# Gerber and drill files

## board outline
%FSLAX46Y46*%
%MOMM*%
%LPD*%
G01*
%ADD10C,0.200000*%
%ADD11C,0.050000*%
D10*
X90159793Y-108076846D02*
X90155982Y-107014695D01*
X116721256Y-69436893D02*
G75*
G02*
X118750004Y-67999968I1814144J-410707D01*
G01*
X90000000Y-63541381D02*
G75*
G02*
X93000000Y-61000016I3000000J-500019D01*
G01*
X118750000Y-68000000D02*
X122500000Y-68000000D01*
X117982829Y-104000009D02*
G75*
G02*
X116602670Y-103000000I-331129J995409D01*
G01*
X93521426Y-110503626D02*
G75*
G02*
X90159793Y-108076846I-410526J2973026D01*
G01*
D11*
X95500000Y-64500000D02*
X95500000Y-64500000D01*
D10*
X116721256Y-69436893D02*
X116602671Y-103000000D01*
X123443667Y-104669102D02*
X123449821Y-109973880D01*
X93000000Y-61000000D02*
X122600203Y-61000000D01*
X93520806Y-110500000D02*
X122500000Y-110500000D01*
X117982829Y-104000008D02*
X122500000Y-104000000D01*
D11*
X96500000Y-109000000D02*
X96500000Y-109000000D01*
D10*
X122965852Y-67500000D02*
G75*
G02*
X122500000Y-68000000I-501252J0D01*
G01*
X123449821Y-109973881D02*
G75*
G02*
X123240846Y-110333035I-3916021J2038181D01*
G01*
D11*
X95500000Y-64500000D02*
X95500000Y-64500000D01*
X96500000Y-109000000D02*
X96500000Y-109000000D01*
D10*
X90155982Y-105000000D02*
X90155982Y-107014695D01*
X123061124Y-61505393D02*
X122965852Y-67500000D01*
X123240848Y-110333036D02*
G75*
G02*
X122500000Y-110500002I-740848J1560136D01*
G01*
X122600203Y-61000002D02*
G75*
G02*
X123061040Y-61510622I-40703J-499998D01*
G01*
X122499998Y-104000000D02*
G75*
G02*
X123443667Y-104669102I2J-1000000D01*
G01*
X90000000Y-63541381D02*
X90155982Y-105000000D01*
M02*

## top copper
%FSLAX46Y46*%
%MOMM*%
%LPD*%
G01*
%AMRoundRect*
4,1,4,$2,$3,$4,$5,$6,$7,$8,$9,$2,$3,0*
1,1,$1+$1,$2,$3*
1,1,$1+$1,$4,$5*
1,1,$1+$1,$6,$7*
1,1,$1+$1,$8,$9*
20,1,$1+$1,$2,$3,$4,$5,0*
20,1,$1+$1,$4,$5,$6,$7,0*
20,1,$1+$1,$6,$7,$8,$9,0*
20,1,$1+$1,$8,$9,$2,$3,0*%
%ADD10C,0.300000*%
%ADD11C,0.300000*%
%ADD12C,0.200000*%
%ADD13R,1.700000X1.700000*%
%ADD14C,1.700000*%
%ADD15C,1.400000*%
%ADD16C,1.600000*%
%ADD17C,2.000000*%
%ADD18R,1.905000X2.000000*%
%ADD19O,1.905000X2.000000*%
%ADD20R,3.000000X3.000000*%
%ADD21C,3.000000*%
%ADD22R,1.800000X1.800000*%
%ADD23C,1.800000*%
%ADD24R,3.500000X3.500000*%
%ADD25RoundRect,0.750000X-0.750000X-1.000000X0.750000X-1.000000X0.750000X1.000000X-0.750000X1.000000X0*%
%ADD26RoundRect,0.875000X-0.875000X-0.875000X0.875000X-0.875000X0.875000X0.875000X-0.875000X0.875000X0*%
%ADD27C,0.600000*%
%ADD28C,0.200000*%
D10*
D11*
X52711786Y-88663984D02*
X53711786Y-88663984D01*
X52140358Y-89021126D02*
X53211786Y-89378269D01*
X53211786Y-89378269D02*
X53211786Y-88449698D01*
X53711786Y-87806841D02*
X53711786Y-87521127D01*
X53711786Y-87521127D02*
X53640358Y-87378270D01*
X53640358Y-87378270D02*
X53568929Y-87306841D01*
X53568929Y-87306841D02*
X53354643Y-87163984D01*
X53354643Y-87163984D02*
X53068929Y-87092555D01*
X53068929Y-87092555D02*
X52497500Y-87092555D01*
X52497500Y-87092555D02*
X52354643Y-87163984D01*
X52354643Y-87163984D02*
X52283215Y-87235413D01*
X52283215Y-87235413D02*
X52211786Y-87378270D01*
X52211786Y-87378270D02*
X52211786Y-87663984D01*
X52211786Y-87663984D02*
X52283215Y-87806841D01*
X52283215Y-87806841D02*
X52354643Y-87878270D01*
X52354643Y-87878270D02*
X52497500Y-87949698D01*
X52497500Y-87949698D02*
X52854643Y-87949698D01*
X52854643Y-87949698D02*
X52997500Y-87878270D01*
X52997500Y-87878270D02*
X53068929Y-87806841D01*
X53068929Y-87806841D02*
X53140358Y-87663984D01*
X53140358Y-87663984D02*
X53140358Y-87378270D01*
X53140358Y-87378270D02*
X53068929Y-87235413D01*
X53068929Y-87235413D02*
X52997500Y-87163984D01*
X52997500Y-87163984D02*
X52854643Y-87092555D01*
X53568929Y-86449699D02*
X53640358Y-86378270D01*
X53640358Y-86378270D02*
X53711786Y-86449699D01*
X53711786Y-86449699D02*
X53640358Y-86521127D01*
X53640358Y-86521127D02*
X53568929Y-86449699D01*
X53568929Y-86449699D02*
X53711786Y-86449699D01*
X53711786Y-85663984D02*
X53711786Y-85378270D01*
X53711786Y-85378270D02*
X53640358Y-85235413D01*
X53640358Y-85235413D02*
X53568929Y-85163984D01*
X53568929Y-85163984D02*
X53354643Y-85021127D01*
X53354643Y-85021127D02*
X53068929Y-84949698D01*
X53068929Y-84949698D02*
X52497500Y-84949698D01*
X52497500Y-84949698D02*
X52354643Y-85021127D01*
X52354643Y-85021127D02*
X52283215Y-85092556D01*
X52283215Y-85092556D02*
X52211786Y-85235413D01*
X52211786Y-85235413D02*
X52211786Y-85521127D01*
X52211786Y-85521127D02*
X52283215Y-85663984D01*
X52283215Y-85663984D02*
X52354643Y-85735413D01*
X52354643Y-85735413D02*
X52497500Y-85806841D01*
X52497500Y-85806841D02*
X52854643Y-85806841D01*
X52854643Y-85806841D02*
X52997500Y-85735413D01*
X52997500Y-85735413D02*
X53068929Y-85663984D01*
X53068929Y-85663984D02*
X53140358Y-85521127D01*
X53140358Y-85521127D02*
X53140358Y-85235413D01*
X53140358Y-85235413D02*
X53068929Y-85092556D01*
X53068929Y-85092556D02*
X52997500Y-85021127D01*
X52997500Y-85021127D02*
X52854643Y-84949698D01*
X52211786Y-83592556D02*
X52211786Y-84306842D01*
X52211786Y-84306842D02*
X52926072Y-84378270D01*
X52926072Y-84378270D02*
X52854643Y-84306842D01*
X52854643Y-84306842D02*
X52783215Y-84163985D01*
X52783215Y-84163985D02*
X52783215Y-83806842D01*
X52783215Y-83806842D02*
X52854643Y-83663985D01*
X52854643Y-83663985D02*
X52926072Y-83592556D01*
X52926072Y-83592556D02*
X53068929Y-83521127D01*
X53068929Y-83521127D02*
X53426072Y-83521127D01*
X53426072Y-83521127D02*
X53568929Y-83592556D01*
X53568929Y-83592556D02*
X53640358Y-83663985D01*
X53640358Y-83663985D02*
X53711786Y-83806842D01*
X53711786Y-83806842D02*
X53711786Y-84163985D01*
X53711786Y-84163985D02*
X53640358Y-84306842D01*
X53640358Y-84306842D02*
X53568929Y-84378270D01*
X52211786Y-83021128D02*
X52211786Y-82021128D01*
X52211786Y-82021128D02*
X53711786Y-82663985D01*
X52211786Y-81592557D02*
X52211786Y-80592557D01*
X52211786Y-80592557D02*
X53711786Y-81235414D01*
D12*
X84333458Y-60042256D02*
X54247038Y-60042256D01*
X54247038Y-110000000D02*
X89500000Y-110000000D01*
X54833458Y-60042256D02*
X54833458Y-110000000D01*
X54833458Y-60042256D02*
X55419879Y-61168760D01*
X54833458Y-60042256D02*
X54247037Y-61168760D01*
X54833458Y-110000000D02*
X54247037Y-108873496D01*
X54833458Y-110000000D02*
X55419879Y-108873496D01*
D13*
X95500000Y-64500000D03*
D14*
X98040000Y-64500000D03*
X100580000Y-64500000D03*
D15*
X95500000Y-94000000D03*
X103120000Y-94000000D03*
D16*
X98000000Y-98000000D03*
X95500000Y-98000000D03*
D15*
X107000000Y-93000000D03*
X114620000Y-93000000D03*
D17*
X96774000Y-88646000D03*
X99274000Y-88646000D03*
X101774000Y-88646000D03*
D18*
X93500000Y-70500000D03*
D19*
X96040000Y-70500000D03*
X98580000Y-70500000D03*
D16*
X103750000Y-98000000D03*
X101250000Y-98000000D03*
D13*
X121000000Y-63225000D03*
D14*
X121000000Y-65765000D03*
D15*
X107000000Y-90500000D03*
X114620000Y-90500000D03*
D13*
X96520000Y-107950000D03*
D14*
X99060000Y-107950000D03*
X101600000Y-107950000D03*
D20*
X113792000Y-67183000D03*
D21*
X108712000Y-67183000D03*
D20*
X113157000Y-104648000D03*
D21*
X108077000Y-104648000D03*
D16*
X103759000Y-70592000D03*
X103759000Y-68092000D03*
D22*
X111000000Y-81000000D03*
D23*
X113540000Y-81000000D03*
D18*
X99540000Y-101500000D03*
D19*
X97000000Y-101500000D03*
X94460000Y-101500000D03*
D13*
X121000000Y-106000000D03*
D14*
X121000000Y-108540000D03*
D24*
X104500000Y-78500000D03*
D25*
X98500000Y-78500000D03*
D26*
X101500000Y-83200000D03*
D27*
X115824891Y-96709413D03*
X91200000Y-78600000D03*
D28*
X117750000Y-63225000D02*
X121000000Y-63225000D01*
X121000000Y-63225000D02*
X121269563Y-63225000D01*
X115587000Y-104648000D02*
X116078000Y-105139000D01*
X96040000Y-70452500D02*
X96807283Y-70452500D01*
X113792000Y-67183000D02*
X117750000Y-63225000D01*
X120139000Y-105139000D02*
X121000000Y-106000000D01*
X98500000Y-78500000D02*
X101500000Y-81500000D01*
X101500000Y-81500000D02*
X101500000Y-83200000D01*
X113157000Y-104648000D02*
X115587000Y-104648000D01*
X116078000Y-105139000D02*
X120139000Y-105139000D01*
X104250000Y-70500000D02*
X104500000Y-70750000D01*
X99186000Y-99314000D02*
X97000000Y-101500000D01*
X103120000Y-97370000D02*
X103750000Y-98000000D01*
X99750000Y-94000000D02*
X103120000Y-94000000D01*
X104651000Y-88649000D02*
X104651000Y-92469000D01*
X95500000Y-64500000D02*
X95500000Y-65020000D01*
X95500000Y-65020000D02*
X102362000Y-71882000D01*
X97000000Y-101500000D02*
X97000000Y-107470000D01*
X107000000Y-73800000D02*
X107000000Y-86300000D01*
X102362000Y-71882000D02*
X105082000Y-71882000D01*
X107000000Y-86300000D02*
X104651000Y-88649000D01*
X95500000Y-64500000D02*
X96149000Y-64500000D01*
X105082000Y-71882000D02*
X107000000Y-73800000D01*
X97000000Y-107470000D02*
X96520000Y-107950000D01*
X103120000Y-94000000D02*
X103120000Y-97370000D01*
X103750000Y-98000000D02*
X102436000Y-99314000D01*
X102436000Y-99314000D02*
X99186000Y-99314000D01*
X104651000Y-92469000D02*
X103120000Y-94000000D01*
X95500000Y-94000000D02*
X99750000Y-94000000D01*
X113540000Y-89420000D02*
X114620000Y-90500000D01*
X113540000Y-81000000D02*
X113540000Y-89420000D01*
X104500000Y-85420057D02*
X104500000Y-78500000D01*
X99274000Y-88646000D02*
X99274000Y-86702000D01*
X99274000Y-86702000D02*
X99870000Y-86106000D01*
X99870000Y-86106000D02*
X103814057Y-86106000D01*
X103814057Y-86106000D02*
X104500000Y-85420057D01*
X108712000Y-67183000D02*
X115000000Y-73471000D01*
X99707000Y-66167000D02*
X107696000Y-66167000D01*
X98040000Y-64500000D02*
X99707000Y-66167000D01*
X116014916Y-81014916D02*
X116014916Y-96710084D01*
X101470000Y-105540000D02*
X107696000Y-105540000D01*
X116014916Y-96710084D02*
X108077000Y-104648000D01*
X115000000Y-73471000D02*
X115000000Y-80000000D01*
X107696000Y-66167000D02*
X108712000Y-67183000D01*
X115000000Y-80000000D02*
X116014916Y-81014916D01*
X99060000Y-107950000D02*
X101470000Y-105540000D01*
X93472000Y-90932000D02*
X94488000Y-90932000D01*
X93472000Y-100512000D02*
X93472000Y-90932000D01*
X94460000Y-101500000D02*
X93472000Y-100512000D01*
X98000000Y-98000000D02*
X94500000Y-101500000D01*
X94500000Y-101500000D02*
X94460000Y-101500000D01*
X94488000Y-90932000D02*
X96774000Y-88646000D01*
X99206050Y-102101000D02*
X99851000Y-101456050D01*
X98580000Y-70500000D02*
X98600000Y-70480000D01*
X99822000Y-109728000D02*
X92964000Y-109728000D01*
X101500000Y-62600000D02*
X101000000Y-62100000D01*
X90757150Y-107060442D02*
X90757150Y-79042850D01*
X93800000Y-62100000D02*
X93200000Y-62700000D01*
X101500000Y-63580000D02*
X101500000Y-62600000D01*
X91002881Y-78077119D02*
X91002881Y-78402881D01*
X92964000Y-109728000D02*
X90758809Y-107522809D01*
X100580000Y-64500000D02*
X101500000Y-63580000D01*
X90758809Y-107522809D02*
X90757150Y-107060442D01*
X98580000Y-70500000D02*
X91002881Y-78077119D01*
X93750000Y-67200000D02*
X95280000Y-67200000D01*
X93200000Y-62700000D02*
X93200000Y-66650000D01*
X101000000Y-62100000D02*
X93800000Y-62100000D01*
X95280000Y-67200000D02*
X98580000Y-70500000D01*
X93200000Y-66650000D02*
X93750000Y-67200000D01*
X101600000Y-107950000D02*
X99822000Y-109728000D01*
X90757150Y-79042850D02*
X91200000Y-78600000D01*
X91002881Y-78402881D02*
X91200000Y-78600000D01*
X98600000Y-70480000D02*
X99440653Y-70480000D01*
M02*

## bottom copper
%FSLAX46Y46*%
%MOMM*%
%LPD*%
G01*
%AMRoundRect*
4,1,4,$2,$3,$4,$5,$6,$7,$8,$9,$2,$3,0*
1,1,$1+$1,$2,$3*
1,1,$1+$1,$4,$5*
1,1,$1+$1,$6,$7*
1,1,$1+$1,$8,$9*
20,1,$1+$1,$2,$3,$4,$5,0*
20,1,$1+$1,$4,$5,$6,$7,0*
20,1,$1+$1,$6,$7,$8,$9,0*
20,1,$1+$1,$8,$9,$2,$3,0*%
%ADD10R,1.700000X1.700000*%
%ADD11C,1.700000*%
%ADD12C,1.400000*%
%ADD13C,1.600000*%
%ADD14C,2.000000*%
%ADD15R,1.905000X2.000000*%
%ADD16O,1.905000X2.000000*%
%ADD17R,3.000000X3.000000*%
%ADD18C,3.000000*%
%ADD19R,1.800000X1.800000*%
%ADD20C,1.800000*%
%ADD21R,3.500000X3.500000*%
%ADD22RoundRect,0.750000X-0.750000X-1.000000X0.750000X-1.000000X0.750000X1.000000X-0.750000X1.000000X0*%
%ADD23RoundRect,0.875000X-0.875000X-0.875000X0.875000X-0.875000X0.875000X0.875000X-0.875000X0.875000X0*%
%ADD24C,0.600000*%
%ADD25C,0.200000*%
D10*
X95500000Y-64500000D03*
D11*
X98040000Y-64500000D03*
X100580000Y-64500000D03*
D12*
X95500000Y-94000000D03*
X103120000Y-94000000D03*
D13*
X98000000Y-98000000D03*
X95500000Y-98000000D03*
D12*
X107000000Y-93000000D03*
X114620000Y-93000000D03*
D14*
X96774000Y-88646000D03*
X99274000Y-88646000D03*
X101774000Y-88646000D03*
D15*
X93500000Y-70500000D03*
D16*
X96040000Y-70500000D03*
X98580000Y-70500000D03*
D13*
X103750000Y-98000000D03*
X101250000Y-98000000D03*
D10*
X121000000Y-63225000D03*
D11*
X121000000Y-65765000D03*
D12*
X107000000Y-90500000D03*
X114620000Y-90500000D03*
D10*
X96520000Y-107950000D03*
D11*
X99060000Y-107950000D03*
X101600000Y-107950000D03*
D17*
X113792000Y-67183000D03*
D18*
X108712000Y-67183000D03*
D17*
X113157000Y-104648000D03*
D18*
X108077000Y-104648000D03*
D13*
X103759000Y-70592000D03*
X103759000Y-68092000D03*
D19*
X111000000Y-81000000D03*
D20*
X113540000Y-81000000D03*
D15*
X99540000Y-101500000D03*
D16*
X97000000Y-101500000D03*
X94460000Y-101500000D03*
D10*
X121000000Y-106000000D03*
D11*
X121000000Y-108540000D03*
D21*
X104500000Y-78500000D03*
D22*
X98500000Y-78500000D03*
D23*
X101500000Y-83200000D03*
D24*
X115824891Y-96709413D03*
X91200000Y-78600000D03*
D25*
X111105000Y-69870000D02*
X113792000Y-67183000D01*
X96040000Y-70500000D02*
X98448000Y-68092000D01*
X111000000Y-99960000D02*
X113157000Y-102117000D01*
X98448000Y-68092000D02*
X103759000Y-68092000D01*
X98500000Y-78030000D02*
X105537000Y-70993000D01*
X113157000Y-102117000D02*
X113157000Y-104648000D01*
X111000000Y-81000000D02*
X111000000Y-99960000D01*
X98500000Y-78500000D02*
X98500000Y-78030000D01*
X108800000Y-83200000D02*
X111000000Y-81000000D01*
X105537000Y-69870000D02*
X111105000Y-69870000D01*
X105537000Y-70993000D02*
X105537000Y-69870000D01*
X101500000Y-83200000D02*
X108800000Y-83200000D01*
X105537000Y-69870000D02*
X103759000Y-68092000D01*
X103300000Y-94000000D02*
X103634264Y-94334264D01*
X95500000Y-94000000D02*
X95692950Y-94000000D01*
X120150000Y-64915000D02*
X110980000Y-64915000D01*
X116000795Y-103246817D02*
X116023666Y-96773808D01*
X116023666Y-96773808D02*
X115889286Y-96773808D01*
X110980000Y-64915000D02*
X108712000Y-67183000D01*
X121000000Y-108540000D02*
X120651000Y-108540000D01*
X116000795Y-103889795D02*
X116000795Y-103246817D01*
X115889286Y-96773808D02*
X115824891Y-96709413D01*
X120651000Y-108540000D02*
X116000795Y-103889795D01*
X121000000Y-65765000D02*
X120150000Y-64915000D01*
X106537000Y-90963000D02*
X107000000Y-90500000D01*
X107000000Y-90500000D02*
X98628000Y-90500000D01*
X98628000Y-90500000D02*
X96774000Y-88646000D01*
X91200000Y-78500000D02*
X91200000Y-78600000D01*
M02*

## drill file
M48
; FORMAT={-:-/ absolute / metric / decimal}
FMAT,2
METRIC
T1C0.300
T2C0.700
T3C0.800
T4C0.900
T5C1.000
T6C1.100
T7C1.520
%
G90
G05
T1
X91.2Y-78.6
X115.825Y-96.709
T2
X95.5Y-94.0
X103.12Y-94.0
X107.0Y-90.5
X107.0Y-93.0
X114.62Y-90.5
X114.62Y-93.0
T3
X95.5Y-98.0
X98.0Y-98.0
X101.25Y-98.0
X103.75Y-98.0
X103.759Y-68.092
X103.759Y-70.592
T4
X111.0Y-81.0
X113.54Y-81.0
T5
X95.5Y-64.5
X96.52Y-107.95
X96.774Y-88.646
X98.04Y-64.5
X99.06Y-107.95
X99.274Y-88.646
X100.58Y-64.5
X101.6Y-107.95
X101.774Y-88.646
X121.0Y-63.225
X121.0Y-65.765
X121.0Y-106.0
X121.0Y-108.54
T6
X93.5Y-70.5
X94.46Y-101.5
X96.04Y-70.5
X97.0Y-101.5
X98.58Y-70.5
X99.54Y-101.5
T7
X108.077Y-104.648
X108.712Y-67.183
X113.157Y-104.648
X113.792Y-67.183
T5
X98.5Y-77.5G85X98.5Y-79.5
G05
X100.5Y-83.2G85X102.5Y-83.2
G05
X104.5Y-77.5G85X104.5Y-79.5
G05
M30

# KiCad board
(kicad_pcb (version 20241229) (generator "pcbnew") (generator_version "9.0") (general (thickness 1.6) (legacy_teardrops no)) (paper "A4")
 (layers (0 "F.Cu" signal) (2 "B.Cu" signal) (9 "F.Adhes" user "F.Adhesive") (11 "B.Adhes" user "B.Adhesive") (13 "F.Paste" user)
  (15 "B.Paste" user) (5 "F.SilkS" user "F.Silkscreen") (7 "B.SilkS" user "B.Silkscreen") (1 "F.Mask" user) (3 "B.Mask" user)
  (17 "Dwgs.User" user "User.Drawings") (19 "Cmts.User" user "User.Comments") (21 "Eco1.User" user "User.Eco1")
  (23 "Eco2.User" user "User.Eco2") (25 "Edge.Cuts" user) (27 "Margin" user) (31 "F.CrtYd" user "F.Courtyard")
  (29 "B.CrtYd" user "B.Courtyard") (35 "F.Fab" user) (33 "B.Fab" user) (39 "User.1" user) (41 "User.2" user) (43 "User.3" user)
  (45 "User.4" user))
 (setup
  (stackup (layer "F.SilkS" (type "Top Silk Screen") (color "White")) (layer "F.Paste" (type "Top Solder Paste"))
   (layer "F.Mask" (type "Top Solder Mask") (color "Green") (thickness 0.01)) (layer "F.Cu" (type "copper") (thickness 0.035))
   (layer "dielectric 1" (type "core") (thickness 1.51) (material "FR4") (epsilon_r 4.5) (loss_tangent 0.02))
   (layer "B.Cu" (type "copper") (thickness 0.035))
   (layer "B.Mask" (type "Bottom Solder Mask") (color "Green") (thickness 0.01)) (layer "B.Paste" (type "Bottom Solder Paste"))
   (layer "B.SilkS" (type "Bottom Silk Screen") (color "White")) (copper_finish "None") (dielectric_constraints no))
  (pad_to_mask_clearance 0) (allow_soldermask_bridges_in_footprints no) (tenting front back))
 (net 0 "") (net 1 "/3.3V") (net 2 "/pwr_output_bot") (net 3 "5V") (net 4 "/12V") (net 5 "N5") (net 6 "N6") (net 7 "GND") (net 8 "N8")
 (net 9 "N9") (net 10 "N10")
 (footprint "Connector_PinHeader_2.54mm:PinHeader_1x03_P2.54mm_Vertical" (layer "F.Cu") (at 95.5 64.5 90)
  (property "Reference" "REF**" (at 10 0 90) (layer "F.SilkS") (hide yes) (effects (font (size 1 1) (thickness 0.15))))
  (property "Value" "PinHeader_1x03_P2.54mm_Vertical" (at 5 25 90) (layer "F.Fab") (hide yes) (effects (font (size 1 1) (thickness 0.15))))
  (pad "1" thru_hole rect (at 0 0 90) (size 1.7 1.7) (drill 1) (layers "*.Cu" "*.Mask") (remove_unused_layers no) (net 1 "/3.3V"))
  (pad "2" thru_hole circle (at 0 2.54 90) (size 1.7 1.7) (drill 1) (layers "*.Cu" "*.Mask") (remove_unused_layers no)
   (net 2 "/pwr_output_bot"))
  (pad "3" thru_hole circle (at 0 5.08 90) (size 1.7 1.7) (drill 1) (layers "*.Cu" "*.Mask") (remove_unused_layers no) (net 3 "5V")))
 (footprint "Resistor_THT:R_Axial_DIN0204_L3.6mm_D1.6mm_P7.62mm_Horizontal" (layer "F.Cu") (at 95.5 94)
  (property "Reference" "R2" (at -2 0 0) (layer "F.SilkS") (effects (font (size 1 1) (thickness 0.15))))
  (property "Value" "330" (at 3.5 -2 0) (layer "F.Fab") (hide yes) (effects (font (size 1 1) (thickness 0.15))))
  (pad "1" thru_hole circle (at 0 0) (size 1.4 1.4) (drill 0.7) (layers "*.Cu" "*.Mask") (remove_unused_layers no) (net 1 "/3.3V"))
  (pad "2" thru_hole circle (at 7.62 0) (size 1.4 1.4) (drill 0.7) (layers "*.Cu" "*.Mask") (remove_unused_layers no) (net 1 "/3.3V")))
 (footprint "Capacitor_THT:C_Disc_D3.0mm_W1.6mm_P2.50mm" (layer "F.Cu") (at 95.5 98)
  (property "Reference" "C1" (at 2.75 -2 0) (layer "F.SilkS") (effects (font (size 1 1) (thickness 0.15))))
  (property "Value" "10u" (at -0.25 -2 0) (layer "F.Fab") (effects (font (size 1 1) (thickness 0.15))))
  (pad "1" thru_hole circle (at 2.5 0) (size 1.6 1.6) (drill 0.8) (layers "*.Cu" "*.Mask") (remove_unused_layers no) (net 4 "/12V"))
  (pad "2" thru_hole circle (at 0 0) (size 1.6 1.6) (drill 0.8) (layers "*.Cu" "*.Mask") (remove_unused_layers no)))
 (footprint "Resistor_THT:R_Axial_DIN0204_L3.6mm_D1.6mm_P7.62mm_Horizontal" (layer "F.Cu") (at 107 93)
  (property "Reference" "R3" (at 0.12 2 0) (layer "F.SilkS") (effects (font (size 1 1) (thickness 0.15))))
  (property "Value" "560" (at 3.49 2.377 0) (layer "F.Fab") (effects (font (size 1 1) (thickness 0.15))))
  (pad "1" thru_hole circle (at 0 0) (size 1.4 1.4) (drill 0.7) (layers "*.Cu" "*.Mask") (remove_unused_layers no))
  (pad "2" thru_hole circle (at 7.62 0) (size 1.4 1.4) (drill 0.7) (layers "*.Cu" "*.Mask") (remove_unused_layers no)))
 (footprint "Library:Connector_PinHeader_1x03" (layer "F.Cu") (at 98.774 92.146)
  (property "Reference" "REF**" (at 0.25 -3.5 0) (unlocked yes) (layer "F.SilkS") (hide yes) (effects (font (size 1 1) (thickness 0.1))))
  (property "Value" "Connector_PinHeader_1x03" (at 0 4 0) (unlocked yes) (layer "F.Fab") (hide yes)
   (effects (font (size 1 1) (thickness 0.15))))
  (pad "1" thru_hole circle (at -2 -3.5) (size 2 2) (drill 1) (layers "*.Cu" "*.Mask") (remove_unused_layers no) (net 4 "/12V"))
  (pad "2" thru_hole circle (at 0.5 -3.5) (size 2 2) (drill 1) (layers "*.Cu" "*.Mask") (remove_unused_layers no) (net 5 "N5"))
  (pad "3" thru_hole circle (at 3 -3.5) (size 2 2) (drill 1) (layers "*.Cu" "*.Mask") (remove_unused_layers no)))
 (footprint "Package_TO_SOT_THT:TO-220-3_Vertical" (layer "F.Cu") (at 93.5 70.5)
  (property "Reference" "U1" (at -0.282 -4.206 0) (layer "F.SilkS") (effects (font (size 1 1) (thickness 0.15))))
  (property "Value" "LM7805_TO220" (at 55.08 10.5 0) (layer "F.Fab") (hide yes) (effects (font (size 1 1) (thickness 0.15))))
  (pad "1" thru_hole rect (at 0 0) (size 1.905 2) (drill 1.1) (layers "*.Cu" "*.Mask") (remove_unused_layers no) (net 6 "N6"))
  (pad "2" thru_hole oval (at 2.54 0) (size 1.905 2) (drill 1.1) (layers "*.Cu" "*.Mask") (remove_unused_layers no) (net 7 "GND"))
  (pad "3" thru_hole oval (at 5.08 0) (size 1.905 2) (drill 1.1) (layers "*.Cu" "*.Mask") (remove_unused_layers no) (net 3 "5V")))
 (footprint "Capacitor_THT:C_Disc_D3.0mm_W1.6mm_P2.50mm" (layer "F.Cu") (at 101.25 98)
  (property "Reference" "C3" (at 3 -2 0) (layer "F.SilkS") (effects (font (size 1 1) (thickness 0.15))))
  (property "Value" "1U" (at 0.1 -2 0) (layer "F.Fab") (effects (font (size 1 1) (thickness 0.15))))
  (pad "1" thru_hole circle (at 2.5 0) (size 1.6 1.6) (drill 0.8) (layers "*.Cu" "*.Mask") (remove_unused_layers no) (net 1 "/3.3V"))
  (pad "2" thru_hole circle (at 0 0) (size 1.6 1.6) (drill 0.8) (layers "*.Cu" "*.Mask") (remove_unused_layers no)))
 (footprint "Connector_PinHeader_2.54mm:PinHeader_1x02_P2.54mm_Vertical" (layer "F.Cu") (at 121 63.225)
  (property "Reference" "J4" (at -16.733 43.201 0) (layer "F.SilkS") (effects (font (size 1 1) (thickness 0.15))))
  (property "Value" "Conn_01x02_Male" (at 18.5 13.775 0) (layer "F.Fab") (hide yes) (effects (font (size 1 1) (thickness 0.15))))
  (pad "1" thru_hole rect (at 0 0) (size 1.7 1.7) (drill 1) (layers "*.Cu" "*.Mask") (remove_unused_layers no) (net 7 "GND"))
  (pad "2" thru_hole circle (at 0 2.54) (size 1.7 1.7) (drill 1) (layers "*.Cu" "*.Mask") (remove_unused_layers no)
   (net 2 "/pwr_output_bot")))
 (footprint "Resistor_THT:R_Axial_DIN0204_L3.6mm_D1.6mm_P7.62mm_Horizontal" (layer "F.Cu") (at 107 90.5)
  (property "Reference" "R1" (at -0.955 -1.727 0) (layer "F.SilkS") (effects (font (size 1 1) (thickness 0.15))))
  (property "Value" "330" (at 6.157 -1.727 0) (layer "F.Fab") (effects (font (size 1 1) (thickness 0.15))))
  (pad "1" thru_hole circle (at 0 0) (size 1.4 1.4) (drill 0.7) (layers "*.Cu" "*.Mask") (remove_unused_layers no) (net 4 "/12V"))
  (pad "2" thru_hole circle (at 7.62 0) (size 1.4 1.4) (drill 0.7) (layers "*.Cu" "*.Mask") (remove_unused_layers no) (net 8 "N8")))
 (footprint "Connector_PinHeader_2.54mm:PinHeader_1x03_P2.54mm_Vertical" (layer "F.Cu") (at 96.52 107.95 90)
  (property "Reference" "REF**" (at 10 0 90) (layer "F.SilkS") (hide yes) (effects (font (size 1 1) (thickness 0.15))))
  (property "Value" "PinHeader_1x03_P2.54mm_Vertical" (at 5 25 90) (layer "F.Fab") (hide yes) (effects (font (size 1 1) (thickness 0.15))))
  (pad "1" thru_hole rect (at 0 0 90) (size 1.7 1.7) (drill 1) (layers "*.Cu" "*.Mask") (remove_unused_layers no) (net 1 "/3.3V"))
  (pad "2" thru_hole circle (at 0 2.54 90) (size 1.7 1.7) (drill 1) (layers "*.Cu" "*.Mask") (remove_unused_layers no)
   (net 2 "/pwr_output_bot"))
  (pad "3" thru_hole circle (at 0 5.08 90) (size 1.7 1.7) (drill 1) (layers "*.Cu" "*.Mask") (remove_unused_layers no) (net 3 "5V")))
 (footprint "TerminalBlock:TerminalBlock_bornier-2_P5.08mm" (layer "F.Cu") (at 113.792 67.183 180)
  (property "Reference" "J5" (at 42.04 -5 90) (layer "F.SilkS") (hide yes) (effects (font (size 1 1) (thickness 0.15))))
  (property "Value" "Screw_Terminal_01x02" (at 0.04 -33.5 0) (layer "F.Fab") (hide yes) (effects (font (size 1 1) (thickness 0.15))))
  (pad "1" thru_hole rect (at 0 0 180) (size 3 3) (drill 1.52) (layers "*.Cu" "*.Mask") (remove_unused_layers no) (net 7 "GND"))
  (pad "2" thru_hole circle (at 5.08 0 180) (size 3 3) (drill 1.52) (layers "*.Cu" "*.Mask") (remove_unused_layers no)
   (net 2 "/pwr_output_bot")))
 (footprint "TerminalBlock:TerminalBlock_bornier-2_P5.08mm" (layer "F.Cu") (at 113.157 104.648 180)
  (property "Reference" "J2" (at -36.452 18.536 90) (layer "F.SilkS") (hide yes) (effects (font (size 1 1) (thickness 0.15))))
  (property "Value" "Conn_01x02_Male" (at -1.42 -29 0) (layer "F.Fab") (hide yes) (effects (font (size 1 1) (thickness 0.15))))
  (pad "1" thru_hole rect (at 0 0 180) (size 3 3) (drill 1.52) (layers "*.Cu" "*.Mask") (remove_unused_layers no) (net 7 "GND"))
  (pad "2" thru_hole circle (at 5.08 0 180) (size 3 3) (drill 1.52) (layers "*.Cu" "*.Mask") (remove_unused_layers no)
   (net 2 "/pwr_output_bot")))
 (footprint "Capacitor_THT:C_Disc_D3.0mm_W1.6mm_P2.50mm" (layer "F.Cu") (at 103.759 70.592 90)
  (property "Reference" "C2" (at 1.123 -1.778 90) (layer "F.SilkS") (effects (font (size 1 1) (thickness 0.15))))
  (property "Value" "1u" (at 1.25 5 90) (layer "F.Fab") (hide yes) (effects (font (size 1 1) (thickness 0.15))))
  (pad "1" thru_hole circle (at 0 0 90) (size 1.6 1.6) (drill 0.8) (layers "*.Cu" "*.Mask") (remove_unused_layers no) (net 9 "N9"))
  (pad "2" thru_hole circle (at 2.5 0 90) (size 1.6 1.6) (drill 0.8) (layers "*.Cu" "*.Mask") (remove_unused_layers no) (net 7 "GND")))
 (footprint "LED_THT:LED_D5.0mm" (layer "F.Cu") (at 111 81)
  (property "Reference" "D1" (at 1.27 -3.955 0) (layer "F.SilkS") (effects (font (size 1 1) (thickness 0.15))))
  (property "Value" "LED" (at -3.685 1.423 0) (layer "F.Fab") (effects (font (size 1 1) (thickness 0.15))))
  (pad "1" thru_hole rect (at 0 0) (size 1.8 1.8) (drill 0.9) (layers "*.Cu" "*.Mask") (remove_unused_layers no) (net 7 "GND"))
  (pad "2" thru_hole circle (at 2.54 0) (size 1.8 1.8) (drill 0.9) (layers "*.Cu" "*.Mask") (remove_unused_layers no) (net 8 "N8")))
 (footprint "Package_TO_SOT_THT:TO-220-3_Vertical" (layer "F.Cu") (at 99.54 101.5 180)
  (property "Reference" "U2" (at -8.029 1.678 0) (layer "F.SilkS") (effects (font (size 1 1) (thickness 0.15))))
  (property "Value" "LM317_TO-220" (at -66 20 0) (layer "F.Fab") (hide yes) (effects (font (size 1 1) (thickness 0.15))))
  (pad "1" thru_hole rect (at 0 0 180) (size 1.905 2) (drill 1.1) (layers "*.Cu" "*.Mask") (remove_unused_layers no) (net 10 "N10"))
  (pad "2" thru_hole oval (at 2.54 0 180) (size 1.905 2) (drill 1.1) (layers "*.Cu" "*.Mask") (remove_unused_layers no) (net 1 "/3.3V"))
  (pad "3" thru_hole oval (at 5.08 0 180) (size 1.905 2) (drill 1.1) (layers "*.Cu" "*.Mask") (remove_unused_layers no) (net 4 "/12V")))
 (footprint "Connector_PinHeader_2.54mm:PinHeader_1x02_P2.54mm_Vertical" (layer "F.Cu") (at 121 106)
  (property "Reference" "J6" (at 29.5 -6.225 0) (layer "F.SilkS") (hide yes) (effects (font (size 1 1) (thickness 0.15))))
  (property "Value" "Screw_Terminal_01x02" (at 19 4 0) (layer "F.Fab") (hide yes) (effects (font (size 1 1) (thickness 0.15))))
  (pad "1" thru_hole rect (at 0 0) (size 1.7 1.7) (drill 1) (layers "*.Cu" "*.Mask") (remove_unused_layers no) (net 7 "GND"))
  (pad "2" thru_hole circle (at 0 2.54) (size 1.7 1.7) (drill 1) (layers "*.Cu" "*.Mask") (remove_unused_layers no)
   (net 2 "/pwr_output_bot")))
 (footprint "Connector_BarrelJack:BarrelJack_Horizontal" (layer "F.Cu") (at 104.5 78.5)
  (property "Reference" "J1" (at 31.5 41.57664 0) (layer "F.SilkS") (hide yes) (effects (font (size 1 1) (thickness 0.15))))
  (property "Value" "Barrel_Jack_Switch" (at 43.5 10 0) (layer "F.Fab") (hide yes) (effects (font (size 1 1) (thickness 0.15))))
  (pad "1" thru_hole rect (at 0 0) (size 3.5 3.5) (drill oval 1 3) (layers "*.Cu" "*.Mask") (remove_unused_layers no) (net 5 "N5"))
  (pad "2" thru_hole roundrect (at -6 0) (size 3 3.5) (drill oval 1 3) (layers "*.Cu" "*.Mask") (remove_unused_layers no)
   (roundrect_rratio 0.25) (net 7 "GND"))
  (pad "3" thru_hole roundrect (at -3 4.7) (size 3.5 3.5) (drill oval 3 1) (layers "*.Cu" "*.Mask") (remove_unused_layers no)
   (roundrect_rratio 0.25) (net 7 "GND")))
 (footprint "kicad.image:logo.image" (layer "B.Cu") (at 110.49 86.106 180)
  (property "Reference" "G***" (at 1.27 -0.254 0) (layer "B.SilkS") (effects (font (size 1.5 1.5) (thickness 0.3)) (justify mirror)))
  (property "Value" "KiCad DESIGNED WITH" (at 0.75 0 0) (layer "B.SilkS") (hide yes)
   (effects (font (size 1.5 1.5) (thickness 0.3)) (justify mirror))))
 (gr_line (start 90.159793 108.076846) (end 90.155982 107.014695) (stroke (width 0.2) (type solid)) (layer "Edge.Cuts"))
 (gr_arc (start 116.721256 69.436893) (mid 117.460312 68.329729) (end 118.75 68) (stroke (width 0.2) (type solid)) (layer "Edge.Cuts"))
 (gr_arc (start 90 63.541381) (mid 91.034128 61.720746) (end 93 61) (stroke (width 0.2) (type solid)) (layer "Edge.Cuts"))
 (gr_line (start 118.75 68) (end 122.5 68) (stroke (width 0.2) (type solid)) (layer "Edge.Cuts"))
 (gr_arc (start 117.982829 104.000009) (mid 117.036207 103.854071) (end 116.60267 103) (stroke (width 0.2) (type solid)) (layer "Edge.Cuts"))
 (gr_arc (start 93.521426 110.503626) (mid 91.354212 109.964005) (end 90.159793 108.076846) (stroke (width 0.2) (type solid))
  (layer "Edge.Cuts"))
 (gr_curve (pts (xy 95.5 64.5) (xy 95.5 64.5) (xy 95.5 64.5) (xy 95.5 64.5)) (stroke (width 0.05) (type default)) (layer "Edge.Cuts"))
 (gr_line (start 116.721256 69.436893) (end 116.602671 103) (stroke (width 0.2) (type solid)) (layer "Edge.Cuts"))
 (gr_line (start 123.443667 104.669102) (end 123.449821 109.97388) (stroke (width 0.2) (type solid)) (layer "Edge.Cuts"))
 (gr_line (start 93 61) (end 122.600203 61) (stroke (width 0.2) (type solid)) (layer "Edge.Cuts"))
 (gr_line (start 93.520806 110.5) (end 122.5 110.5) (stroke (width 0.2) (type solid)) (layer "Edge.Cuts"))
 (gr_line (start 117.982829 104.000008) (end 122.5 104) (stroke (width 0.2) (type solid)) (layer "Edge.Cuts"))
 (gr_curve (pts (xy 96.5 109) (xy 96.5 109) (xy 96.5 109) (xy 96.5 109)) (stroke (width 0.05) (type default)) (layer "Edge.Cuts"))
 (gr_arc (start 122.965852 67.5) (mid 122.831341 67.841694) (end 122.5 68) (stroke (width 0.2) (type solid)) (layer "Edge.Cuts"))
 (gr_arc (start 123.449821 109.973881) (mid 123.34956 110.155917) (end 123.240843 110.333033) (stroke (width 0.2) (type solid))
  (layer "Edge.Cuts"))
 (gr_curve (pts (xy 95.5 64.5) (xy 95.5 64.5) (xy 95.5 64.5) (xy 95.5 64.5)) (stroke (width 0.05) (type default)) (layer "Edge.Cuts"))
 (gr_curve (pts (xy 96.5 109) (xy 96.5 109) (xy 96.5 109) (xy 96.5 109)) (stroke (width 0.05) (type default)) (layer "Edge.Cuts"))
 (gr_line (start 90.155982 105) (end 90.155982 107.014695) (stroke (width 0.2) (type solid)) (layer "Edge.Cuts"))
 (gr_line (start 123.061124 61.505393) (end 122.965852 67.5) (stroke (width 0.2) (type solid)) (layer "Edge.Cuts"))
 (gr_arc (start 123.240848 110.333036) (mid 122.879715 110.457742) (end 122.5 110.5) (stroke (width 0.2) (type solid)) (layer "Edge.Cuts"))
 (gr_arc (start 122.600203 61.000002) (mid 122.931911 61.163898) (end 123.06104 61.510622) (stroke (width 0.2) (type solid))
  (layer "Edge.Cuts"))
 (gr_arc (start 122.499998 104) (mid 123.078403 104.184249) (end 123.443667 104.669102) (stroke (width 0.2) (type solid))
  (layer "Edge.Cuts"))
 (gr_line (start 90 63.541381) (end 90.155982 105) (stroke (width 0.2) (type solid)) (layer "Edge.Cuts"))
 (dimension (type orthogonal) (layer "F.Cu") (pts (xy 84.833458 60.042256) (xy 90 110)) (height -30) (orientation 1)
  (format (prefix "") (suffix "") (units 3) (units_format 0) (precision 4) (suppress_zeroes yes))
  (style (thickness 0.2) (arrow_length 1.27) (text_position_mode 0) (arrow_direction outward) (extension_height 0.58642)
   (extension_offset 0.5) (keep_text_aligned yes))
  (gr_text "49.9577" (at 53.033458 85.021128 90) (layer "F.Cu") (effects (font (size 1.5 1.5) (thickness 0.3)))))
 (segment (start 117.75 63.225) (end 121 63.225) (width 0.2) (layer "F.Cu") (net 7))
 (segment (start 121 63.225) (end 121.269563 63.225) (width 0.2) (layer "F.Cu") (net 7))
 (segment (start 115.587 104.648) (end 116.078 105.139) (width 0.2) (layer "F.Cu") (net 7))
 (segment (start 96.04 70.4525) (end 96.807283 70.4525) (width 0.2) (layer "F.Cu") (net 7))
 (segment (start 113.792 67.183) (end 117.75 63.225) (width 0.2) (layer "F.Cu") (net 7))
 (segment (start 120.139 105.139) (end 121 106) (width 0.2) (layer "F.Cu") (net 7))
 (segment (start 98.5 78.5) (end 101.5 81.5) (width 0.2) (layer "F.Cu") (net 7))
 (segment (start 101.5 81.5) (end 101.5 83.2) (width 0.2) (layer "F.Cu") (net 7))
 (segment (start 113.157 104.648) (end 115.587 104.648) (width 0.2) (layer "F.Cu") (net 7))
 (segment (start 116.078 105.139) (end 120.139 105.139) (width 0.2) (layer "F.Cu") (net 7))
 (segment (start 111.105 69.87) (end 113.792 67.183) (width 0.2) (layer "B.Cu") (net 7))
 (segment (start 96.04 70.5) (end 98.448 68.092) (width 0.2) (layer "B.Cu") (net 7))
 (segment (start 111 99.96) (end 113.157 102.117) (width 0.2) (layer "B.Cu") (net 7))
 (segment (start 98.448 68.092) (end 103.759 68.092) (width 0.2) (layer "B.Cu") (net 7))
 (segment (start 98.5 78.03) (end 105.537 70.993) (width 0.2) (layer "B.Cu") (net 7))
 (segment (start 113.157 102.117) (end 113.157 104.648) (width 0.2) (layer "B.Cu") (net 7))
 (segment (start 111 81) (end 111 99.96) (width 0.2) (layer "B.Cu") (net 7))
 (segment (start 98.5 78.5) (end 98.5 78.03) (width 0.2) (layer "B.Cu") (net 7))
 (segment (start 108.8 83.2) (end 111 81) (width 0.2) (layer "B.Cu") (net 7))
 (segment (start 105.537 69.87) (end 111.105 69.87) (width 0.2) (layer "B.Cu") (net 7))
 (segment (start 105.537 70.993) (end 105.537 69.87) (width 0.2) (layer "B.Cu") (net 7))
 (segment (start 101.5 83.2) (end 108.8 83.2) (width 0.2) (layer "B.Cu") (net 7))
 (segment (start 105.537 69.87) (end 103.759 68.092) (width 0.2) (layer "B.Cu") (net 7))
 (segment (start 104.25 70.5) (end 104.5 70.75) (width 0.2) (layer "F.Cu") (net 9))
 (segment (start 99.186 99.314) (end 97 101.5) (width 0.2) (layer "F.Cu") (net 1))
 (segment (start 103.12 97.37) (end 103.75 98) (width 0.2) (layer "F.Cu") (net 1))
 (segment (start 99.75 94) (end 103.12 94) (width 0.2) (layer "F.Cu") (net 1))
 (segment (start 104.651 88.649) (end 104.651 92.469) (width 0.2) (layer "F.Cu") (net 1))
 (segment (start 95.5 64.5) (end 95.5 65.02) (width 0.2) (layer "F.Cu") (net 1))
 (segment (start 95.5 65.02) (end 102.362 71.882) (width 0.2) (layer "F.Cu") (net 1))
 (segment (start 97 101.5) (end 97 107.47) (width 0.2) (layer "F.Cu") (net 1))
 (segment (start 107 73.8) (end 107 86.3) (width 0.2) (layer "F.Cu") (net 1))
 (segment (start 102.362 71.882) (end 105.082 71.882) (width 0.2) (layer "F.Cu") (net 1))
 (segment (start 107 86.3) (end 104.651 88.649) (width 0.2) (layer "F.Cu") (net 1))
 (segment (start 95.5 64.5) (end 96.149 64.5) (width 0.2) (layer "F.Cu") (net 1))
 (segment (start 105.082 71.882) (end 107 73.8) (width 0.2) (layer "F.Cu") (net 1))
 (segment (start 97 107.47) (end 96.52 107.95) (width 0.2) (layer "F.Cu") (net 1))
 (segment (start 103.12 94) (end 103.12 97.37) (width 0.2) (layer "F.Cu") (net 1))
 (segment (start 103.75 98) (end 102.436 99.314) (width 0.2) (layer "F.Cu") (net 1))
 (segment (start 102.436 99.314) (end 99.186 99.314) (width 0.2) (layer "F.Cu") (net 1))
 (segment (start 104.651 92.469) (end 103.12 94) (width 0.2) (layer "F.Cu") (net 1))
 (segment (start 95.5 94) (end 99.75 94) (width 0.2) (layer "F.Cu") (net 1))
 (segment (start 103.3 94) (end 103.634264 94.334264) (width 0.2) (layer "B.Cu") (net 1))
 (segment (start 95.5 94) (end 95.69295 94) (width 0.2) (layer "B.Cu") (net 1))
 (segment (start 113.54 89.42) (end 114.62 90.5) (width 0.2) (layer "F.Cu") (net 8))
 (segment (start 113.54 81) (end 113.54 89.42) (width 0.2) (layer "F.Cu") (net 8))
 (segment (start 104.5 85.420057) (end 104.5 78.5) (width 0.2) (layer "F.Cu") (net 5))
 (segment (start 99.274 88.646) (end 99.274 86.702) (width 0.2) (layer "F.Cu") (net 5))
 (segment (start 99.274 86.702) (end 99.87 86.106) (width 0.2) (layer "F.Cu") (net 5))
 (segment (start 99.87 86.106) (end 103.814057 86.106) (width 0.2) (layer "F.Cu") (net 5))
 (segment (start 103.814057 86.106) (end 104.5 85.420057) (width 0.2) (layer "F.Cu") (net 5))
 (segment (start 108.712 67.183) (end 115 73.471) (width 0.2) (layer "F.Cu") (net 2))
 (segment (start 99.707 66.167) (end 107.696 66.167) (width 0.2) (layer "F.Cu") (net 2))
 (segment (start 98.04 64.5) (end 99.707 66.167) (width 0.2) (layer "F.Cu") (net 2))
 (segment (start 116.014916 81.014916) (end 116.014916 96.710084) (width 0.2) (layer "F.Cu") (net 2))
 (segment (start 101.47 105.54) (end 107.696 105.54) (width 0.2) (layer "F.Cu") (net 2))
 (segment (start 116.014916 96.710084) (end 108.077 104.648) (width 0.2) (layer "F.Cu") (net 2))
 (segment (start 115 73.471) (end 115 80) (width 0.2) (layer "F.Cu") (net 2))
 (segment (start 107.696 66.167) (end 108.712 67.183) (width 0.2) (layer "F.Cu") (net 2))
 (segment (start 115 80) (end 116.014916 81.014916) (width 0.2) (layer "F.Cu") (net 2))
 (segment (start 99.06 107.95) (end 101.47 105.54) (width 0.2) (layer "F.Cu") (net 2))
 (via (at 115.824891 96.709413) (size 0.6) (drill 0.3) (layers "F.Cu" "B.Cu") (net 2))
 (segment (start 120.15 64.915) (end 110.98 64.915) (width 0.2) (layer "B.Cu") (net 2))
 (segment (start 116.000795 103.246817) (end 116.023666 96.773808) (width 0.2) (layer "B.Cu") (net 2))
 (segment (start 116.023666 96.773808) (end 115.889286 96.773808) (width 0.2) (layer "B.Cu") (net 2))
 (segment (start 110.98 64.915) (end 108.712 67.183) (width 0.2) (layer "B.Cu") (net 2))
 (segment (start 121 108.54) (end 120.651 108.54) (width 0.2) (layer "B.Cu") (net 2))
 (segment (start 116.000795 103.889795) (end 116.000795 103.246817) (width 0.2) (layer "B.Cu") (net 2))
 (segment (start 115.889286 96.773808) (end 115.824891 96.709413) (width 0.2) (layer "B.Cu") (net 2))
 (segment (start 120.651 108.54) (end 116.000795 103.889795) (width 0.2) (layer "B.Cu") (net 2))
 (segment (start 121 65.765) (end 120.15 64.915) (width 0.2) (layer "B.Cu") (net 2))
 (segment (start 93.472 90.932) (end 94.488 90.932) (width 0.2) (layer "F.Cu") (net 4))
 (segment (start 93.472 100.512) (end 93.472 90.932) (width 0.2) (layer "F.Cu") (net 4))
 (segment (start 94.46 101.5) (end 93.472 100.512) (width 0.2) (layer "F.Cu") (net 4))
 (segment (start 98 98) (end 94.5 101.5) (width 0.2) (layer "F.Cu") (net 4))
 (segment (start 94.5 101.5) (end 94.46 101.5) (width 0.2) (layer "F.Cu") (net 4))
 (segment (start 94.488 90.932) (end 96.774 88.646) (width 0.2) (layer "F.Cu") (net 4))
 (segment (start 106.537 90.963) (end 107 90.5) (width 0.2) (layer "B.Cu") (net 4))
 (segment (start 107 90.5) (end 98.628 90.5) (width 0.2) (layer "B.Cu") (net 4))
 (segment (start 98.628 90.5) (end 96.774 88.646) (width 0.2) (layer "B.Cu") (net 4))
 (segment (start 99.20605 102.101) (end 99.851 101.45605) (width 0.2) (layer "F.Cu") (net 10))
 (segment (start 98.58 70.5) (end 98.6 70.48) (width 0.2) (layer "F.Cu") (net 3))
 (segment (start 99.822 109.728) (end 92.964 109.728) (width 0.2) (layer "F.Cu") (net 3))
 (segment (start 101.5 62.6) (end 101 62.1) (width 0.2) (layer "F.Cu") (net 3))
 (segment (start 90.75715 107.060442) (end 90.75715 79.04285) (width 0.2) (layer "F.Cu") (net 3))
 (segment (start 93.8 62.1) (end 93.2 62.7) (width 0.2) (layer "F.Cu") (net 3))
 (segment (start 101.5 63.58) (end 101.5 62.6) (width 0.2) (layer "F.Cu") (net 3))
 (segment (start 91.002881 78.077119) (end 91.002881 78.402881) (width 0.2) (layer "F.Cu") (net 3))
 (segment (start 92.964 109.728) (end 90.758809 107.522809) (width 0.2) (layer "F.Cu") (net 3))
 (segment (start 100.58 64.5) (end 101.5 63.58) (width 0.2) (layer "F.Cu") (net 3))
 (segment (start 90.758809 107.522809) (end 90.75715 107.060442) (width 0.2) (layer "F.Cu") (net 3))
 (segment (start 98.58 70.5) (end 91.002881 78.077119) (width 0.2) (layer "F.Cu") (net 3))
 (segment (start 93.75 67.2) (end 95.28 67.2) (width 0.2) (layer "F.Cu") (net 3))
 (segment (start 93.2 62.7) (end 93.2 66.65) (width 0.2) (layer "F.Cu") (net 3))
 (segment (start 101 62.1) (end 93.8 62.1) (width 0.2) (layer "F.Cu") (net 3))
 (segment (start 95.28 67.2) (end 98.58 70.5) (width 0.2) (layer "F.Cu") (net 3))
 (segment (start 93.2 66.65) (end 93.75 67.2) (width 0.2) (layer "F.Cu") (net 3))
 (segment (start 101.6 107.95) (end 99.822 109.728) (width 0.2) (layer "F.Cu") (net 3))
 (segment (start 90.75715 79.04285) (end 91.2 78.6) (width 0.2) (layer "F.Cu") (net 3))
 (segment (start 91.002881 78.402881) (end 91.2 78.6) (width 0.2) (layer "F.Cu") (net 3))
 (segment (start 98.6 70.48) (end 99.440653 70.48) (width 0.2) (layer "F.Cu") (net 3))
 (via (at 91.2 78.6) (size 0.6) (drill 0.3) (layers "F.Cu" "B.Cu") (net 3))
 (segment (start 91.2 78.5) (end 91.2 78.6) (width 0.2) (layer "B.Cu") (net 3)))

